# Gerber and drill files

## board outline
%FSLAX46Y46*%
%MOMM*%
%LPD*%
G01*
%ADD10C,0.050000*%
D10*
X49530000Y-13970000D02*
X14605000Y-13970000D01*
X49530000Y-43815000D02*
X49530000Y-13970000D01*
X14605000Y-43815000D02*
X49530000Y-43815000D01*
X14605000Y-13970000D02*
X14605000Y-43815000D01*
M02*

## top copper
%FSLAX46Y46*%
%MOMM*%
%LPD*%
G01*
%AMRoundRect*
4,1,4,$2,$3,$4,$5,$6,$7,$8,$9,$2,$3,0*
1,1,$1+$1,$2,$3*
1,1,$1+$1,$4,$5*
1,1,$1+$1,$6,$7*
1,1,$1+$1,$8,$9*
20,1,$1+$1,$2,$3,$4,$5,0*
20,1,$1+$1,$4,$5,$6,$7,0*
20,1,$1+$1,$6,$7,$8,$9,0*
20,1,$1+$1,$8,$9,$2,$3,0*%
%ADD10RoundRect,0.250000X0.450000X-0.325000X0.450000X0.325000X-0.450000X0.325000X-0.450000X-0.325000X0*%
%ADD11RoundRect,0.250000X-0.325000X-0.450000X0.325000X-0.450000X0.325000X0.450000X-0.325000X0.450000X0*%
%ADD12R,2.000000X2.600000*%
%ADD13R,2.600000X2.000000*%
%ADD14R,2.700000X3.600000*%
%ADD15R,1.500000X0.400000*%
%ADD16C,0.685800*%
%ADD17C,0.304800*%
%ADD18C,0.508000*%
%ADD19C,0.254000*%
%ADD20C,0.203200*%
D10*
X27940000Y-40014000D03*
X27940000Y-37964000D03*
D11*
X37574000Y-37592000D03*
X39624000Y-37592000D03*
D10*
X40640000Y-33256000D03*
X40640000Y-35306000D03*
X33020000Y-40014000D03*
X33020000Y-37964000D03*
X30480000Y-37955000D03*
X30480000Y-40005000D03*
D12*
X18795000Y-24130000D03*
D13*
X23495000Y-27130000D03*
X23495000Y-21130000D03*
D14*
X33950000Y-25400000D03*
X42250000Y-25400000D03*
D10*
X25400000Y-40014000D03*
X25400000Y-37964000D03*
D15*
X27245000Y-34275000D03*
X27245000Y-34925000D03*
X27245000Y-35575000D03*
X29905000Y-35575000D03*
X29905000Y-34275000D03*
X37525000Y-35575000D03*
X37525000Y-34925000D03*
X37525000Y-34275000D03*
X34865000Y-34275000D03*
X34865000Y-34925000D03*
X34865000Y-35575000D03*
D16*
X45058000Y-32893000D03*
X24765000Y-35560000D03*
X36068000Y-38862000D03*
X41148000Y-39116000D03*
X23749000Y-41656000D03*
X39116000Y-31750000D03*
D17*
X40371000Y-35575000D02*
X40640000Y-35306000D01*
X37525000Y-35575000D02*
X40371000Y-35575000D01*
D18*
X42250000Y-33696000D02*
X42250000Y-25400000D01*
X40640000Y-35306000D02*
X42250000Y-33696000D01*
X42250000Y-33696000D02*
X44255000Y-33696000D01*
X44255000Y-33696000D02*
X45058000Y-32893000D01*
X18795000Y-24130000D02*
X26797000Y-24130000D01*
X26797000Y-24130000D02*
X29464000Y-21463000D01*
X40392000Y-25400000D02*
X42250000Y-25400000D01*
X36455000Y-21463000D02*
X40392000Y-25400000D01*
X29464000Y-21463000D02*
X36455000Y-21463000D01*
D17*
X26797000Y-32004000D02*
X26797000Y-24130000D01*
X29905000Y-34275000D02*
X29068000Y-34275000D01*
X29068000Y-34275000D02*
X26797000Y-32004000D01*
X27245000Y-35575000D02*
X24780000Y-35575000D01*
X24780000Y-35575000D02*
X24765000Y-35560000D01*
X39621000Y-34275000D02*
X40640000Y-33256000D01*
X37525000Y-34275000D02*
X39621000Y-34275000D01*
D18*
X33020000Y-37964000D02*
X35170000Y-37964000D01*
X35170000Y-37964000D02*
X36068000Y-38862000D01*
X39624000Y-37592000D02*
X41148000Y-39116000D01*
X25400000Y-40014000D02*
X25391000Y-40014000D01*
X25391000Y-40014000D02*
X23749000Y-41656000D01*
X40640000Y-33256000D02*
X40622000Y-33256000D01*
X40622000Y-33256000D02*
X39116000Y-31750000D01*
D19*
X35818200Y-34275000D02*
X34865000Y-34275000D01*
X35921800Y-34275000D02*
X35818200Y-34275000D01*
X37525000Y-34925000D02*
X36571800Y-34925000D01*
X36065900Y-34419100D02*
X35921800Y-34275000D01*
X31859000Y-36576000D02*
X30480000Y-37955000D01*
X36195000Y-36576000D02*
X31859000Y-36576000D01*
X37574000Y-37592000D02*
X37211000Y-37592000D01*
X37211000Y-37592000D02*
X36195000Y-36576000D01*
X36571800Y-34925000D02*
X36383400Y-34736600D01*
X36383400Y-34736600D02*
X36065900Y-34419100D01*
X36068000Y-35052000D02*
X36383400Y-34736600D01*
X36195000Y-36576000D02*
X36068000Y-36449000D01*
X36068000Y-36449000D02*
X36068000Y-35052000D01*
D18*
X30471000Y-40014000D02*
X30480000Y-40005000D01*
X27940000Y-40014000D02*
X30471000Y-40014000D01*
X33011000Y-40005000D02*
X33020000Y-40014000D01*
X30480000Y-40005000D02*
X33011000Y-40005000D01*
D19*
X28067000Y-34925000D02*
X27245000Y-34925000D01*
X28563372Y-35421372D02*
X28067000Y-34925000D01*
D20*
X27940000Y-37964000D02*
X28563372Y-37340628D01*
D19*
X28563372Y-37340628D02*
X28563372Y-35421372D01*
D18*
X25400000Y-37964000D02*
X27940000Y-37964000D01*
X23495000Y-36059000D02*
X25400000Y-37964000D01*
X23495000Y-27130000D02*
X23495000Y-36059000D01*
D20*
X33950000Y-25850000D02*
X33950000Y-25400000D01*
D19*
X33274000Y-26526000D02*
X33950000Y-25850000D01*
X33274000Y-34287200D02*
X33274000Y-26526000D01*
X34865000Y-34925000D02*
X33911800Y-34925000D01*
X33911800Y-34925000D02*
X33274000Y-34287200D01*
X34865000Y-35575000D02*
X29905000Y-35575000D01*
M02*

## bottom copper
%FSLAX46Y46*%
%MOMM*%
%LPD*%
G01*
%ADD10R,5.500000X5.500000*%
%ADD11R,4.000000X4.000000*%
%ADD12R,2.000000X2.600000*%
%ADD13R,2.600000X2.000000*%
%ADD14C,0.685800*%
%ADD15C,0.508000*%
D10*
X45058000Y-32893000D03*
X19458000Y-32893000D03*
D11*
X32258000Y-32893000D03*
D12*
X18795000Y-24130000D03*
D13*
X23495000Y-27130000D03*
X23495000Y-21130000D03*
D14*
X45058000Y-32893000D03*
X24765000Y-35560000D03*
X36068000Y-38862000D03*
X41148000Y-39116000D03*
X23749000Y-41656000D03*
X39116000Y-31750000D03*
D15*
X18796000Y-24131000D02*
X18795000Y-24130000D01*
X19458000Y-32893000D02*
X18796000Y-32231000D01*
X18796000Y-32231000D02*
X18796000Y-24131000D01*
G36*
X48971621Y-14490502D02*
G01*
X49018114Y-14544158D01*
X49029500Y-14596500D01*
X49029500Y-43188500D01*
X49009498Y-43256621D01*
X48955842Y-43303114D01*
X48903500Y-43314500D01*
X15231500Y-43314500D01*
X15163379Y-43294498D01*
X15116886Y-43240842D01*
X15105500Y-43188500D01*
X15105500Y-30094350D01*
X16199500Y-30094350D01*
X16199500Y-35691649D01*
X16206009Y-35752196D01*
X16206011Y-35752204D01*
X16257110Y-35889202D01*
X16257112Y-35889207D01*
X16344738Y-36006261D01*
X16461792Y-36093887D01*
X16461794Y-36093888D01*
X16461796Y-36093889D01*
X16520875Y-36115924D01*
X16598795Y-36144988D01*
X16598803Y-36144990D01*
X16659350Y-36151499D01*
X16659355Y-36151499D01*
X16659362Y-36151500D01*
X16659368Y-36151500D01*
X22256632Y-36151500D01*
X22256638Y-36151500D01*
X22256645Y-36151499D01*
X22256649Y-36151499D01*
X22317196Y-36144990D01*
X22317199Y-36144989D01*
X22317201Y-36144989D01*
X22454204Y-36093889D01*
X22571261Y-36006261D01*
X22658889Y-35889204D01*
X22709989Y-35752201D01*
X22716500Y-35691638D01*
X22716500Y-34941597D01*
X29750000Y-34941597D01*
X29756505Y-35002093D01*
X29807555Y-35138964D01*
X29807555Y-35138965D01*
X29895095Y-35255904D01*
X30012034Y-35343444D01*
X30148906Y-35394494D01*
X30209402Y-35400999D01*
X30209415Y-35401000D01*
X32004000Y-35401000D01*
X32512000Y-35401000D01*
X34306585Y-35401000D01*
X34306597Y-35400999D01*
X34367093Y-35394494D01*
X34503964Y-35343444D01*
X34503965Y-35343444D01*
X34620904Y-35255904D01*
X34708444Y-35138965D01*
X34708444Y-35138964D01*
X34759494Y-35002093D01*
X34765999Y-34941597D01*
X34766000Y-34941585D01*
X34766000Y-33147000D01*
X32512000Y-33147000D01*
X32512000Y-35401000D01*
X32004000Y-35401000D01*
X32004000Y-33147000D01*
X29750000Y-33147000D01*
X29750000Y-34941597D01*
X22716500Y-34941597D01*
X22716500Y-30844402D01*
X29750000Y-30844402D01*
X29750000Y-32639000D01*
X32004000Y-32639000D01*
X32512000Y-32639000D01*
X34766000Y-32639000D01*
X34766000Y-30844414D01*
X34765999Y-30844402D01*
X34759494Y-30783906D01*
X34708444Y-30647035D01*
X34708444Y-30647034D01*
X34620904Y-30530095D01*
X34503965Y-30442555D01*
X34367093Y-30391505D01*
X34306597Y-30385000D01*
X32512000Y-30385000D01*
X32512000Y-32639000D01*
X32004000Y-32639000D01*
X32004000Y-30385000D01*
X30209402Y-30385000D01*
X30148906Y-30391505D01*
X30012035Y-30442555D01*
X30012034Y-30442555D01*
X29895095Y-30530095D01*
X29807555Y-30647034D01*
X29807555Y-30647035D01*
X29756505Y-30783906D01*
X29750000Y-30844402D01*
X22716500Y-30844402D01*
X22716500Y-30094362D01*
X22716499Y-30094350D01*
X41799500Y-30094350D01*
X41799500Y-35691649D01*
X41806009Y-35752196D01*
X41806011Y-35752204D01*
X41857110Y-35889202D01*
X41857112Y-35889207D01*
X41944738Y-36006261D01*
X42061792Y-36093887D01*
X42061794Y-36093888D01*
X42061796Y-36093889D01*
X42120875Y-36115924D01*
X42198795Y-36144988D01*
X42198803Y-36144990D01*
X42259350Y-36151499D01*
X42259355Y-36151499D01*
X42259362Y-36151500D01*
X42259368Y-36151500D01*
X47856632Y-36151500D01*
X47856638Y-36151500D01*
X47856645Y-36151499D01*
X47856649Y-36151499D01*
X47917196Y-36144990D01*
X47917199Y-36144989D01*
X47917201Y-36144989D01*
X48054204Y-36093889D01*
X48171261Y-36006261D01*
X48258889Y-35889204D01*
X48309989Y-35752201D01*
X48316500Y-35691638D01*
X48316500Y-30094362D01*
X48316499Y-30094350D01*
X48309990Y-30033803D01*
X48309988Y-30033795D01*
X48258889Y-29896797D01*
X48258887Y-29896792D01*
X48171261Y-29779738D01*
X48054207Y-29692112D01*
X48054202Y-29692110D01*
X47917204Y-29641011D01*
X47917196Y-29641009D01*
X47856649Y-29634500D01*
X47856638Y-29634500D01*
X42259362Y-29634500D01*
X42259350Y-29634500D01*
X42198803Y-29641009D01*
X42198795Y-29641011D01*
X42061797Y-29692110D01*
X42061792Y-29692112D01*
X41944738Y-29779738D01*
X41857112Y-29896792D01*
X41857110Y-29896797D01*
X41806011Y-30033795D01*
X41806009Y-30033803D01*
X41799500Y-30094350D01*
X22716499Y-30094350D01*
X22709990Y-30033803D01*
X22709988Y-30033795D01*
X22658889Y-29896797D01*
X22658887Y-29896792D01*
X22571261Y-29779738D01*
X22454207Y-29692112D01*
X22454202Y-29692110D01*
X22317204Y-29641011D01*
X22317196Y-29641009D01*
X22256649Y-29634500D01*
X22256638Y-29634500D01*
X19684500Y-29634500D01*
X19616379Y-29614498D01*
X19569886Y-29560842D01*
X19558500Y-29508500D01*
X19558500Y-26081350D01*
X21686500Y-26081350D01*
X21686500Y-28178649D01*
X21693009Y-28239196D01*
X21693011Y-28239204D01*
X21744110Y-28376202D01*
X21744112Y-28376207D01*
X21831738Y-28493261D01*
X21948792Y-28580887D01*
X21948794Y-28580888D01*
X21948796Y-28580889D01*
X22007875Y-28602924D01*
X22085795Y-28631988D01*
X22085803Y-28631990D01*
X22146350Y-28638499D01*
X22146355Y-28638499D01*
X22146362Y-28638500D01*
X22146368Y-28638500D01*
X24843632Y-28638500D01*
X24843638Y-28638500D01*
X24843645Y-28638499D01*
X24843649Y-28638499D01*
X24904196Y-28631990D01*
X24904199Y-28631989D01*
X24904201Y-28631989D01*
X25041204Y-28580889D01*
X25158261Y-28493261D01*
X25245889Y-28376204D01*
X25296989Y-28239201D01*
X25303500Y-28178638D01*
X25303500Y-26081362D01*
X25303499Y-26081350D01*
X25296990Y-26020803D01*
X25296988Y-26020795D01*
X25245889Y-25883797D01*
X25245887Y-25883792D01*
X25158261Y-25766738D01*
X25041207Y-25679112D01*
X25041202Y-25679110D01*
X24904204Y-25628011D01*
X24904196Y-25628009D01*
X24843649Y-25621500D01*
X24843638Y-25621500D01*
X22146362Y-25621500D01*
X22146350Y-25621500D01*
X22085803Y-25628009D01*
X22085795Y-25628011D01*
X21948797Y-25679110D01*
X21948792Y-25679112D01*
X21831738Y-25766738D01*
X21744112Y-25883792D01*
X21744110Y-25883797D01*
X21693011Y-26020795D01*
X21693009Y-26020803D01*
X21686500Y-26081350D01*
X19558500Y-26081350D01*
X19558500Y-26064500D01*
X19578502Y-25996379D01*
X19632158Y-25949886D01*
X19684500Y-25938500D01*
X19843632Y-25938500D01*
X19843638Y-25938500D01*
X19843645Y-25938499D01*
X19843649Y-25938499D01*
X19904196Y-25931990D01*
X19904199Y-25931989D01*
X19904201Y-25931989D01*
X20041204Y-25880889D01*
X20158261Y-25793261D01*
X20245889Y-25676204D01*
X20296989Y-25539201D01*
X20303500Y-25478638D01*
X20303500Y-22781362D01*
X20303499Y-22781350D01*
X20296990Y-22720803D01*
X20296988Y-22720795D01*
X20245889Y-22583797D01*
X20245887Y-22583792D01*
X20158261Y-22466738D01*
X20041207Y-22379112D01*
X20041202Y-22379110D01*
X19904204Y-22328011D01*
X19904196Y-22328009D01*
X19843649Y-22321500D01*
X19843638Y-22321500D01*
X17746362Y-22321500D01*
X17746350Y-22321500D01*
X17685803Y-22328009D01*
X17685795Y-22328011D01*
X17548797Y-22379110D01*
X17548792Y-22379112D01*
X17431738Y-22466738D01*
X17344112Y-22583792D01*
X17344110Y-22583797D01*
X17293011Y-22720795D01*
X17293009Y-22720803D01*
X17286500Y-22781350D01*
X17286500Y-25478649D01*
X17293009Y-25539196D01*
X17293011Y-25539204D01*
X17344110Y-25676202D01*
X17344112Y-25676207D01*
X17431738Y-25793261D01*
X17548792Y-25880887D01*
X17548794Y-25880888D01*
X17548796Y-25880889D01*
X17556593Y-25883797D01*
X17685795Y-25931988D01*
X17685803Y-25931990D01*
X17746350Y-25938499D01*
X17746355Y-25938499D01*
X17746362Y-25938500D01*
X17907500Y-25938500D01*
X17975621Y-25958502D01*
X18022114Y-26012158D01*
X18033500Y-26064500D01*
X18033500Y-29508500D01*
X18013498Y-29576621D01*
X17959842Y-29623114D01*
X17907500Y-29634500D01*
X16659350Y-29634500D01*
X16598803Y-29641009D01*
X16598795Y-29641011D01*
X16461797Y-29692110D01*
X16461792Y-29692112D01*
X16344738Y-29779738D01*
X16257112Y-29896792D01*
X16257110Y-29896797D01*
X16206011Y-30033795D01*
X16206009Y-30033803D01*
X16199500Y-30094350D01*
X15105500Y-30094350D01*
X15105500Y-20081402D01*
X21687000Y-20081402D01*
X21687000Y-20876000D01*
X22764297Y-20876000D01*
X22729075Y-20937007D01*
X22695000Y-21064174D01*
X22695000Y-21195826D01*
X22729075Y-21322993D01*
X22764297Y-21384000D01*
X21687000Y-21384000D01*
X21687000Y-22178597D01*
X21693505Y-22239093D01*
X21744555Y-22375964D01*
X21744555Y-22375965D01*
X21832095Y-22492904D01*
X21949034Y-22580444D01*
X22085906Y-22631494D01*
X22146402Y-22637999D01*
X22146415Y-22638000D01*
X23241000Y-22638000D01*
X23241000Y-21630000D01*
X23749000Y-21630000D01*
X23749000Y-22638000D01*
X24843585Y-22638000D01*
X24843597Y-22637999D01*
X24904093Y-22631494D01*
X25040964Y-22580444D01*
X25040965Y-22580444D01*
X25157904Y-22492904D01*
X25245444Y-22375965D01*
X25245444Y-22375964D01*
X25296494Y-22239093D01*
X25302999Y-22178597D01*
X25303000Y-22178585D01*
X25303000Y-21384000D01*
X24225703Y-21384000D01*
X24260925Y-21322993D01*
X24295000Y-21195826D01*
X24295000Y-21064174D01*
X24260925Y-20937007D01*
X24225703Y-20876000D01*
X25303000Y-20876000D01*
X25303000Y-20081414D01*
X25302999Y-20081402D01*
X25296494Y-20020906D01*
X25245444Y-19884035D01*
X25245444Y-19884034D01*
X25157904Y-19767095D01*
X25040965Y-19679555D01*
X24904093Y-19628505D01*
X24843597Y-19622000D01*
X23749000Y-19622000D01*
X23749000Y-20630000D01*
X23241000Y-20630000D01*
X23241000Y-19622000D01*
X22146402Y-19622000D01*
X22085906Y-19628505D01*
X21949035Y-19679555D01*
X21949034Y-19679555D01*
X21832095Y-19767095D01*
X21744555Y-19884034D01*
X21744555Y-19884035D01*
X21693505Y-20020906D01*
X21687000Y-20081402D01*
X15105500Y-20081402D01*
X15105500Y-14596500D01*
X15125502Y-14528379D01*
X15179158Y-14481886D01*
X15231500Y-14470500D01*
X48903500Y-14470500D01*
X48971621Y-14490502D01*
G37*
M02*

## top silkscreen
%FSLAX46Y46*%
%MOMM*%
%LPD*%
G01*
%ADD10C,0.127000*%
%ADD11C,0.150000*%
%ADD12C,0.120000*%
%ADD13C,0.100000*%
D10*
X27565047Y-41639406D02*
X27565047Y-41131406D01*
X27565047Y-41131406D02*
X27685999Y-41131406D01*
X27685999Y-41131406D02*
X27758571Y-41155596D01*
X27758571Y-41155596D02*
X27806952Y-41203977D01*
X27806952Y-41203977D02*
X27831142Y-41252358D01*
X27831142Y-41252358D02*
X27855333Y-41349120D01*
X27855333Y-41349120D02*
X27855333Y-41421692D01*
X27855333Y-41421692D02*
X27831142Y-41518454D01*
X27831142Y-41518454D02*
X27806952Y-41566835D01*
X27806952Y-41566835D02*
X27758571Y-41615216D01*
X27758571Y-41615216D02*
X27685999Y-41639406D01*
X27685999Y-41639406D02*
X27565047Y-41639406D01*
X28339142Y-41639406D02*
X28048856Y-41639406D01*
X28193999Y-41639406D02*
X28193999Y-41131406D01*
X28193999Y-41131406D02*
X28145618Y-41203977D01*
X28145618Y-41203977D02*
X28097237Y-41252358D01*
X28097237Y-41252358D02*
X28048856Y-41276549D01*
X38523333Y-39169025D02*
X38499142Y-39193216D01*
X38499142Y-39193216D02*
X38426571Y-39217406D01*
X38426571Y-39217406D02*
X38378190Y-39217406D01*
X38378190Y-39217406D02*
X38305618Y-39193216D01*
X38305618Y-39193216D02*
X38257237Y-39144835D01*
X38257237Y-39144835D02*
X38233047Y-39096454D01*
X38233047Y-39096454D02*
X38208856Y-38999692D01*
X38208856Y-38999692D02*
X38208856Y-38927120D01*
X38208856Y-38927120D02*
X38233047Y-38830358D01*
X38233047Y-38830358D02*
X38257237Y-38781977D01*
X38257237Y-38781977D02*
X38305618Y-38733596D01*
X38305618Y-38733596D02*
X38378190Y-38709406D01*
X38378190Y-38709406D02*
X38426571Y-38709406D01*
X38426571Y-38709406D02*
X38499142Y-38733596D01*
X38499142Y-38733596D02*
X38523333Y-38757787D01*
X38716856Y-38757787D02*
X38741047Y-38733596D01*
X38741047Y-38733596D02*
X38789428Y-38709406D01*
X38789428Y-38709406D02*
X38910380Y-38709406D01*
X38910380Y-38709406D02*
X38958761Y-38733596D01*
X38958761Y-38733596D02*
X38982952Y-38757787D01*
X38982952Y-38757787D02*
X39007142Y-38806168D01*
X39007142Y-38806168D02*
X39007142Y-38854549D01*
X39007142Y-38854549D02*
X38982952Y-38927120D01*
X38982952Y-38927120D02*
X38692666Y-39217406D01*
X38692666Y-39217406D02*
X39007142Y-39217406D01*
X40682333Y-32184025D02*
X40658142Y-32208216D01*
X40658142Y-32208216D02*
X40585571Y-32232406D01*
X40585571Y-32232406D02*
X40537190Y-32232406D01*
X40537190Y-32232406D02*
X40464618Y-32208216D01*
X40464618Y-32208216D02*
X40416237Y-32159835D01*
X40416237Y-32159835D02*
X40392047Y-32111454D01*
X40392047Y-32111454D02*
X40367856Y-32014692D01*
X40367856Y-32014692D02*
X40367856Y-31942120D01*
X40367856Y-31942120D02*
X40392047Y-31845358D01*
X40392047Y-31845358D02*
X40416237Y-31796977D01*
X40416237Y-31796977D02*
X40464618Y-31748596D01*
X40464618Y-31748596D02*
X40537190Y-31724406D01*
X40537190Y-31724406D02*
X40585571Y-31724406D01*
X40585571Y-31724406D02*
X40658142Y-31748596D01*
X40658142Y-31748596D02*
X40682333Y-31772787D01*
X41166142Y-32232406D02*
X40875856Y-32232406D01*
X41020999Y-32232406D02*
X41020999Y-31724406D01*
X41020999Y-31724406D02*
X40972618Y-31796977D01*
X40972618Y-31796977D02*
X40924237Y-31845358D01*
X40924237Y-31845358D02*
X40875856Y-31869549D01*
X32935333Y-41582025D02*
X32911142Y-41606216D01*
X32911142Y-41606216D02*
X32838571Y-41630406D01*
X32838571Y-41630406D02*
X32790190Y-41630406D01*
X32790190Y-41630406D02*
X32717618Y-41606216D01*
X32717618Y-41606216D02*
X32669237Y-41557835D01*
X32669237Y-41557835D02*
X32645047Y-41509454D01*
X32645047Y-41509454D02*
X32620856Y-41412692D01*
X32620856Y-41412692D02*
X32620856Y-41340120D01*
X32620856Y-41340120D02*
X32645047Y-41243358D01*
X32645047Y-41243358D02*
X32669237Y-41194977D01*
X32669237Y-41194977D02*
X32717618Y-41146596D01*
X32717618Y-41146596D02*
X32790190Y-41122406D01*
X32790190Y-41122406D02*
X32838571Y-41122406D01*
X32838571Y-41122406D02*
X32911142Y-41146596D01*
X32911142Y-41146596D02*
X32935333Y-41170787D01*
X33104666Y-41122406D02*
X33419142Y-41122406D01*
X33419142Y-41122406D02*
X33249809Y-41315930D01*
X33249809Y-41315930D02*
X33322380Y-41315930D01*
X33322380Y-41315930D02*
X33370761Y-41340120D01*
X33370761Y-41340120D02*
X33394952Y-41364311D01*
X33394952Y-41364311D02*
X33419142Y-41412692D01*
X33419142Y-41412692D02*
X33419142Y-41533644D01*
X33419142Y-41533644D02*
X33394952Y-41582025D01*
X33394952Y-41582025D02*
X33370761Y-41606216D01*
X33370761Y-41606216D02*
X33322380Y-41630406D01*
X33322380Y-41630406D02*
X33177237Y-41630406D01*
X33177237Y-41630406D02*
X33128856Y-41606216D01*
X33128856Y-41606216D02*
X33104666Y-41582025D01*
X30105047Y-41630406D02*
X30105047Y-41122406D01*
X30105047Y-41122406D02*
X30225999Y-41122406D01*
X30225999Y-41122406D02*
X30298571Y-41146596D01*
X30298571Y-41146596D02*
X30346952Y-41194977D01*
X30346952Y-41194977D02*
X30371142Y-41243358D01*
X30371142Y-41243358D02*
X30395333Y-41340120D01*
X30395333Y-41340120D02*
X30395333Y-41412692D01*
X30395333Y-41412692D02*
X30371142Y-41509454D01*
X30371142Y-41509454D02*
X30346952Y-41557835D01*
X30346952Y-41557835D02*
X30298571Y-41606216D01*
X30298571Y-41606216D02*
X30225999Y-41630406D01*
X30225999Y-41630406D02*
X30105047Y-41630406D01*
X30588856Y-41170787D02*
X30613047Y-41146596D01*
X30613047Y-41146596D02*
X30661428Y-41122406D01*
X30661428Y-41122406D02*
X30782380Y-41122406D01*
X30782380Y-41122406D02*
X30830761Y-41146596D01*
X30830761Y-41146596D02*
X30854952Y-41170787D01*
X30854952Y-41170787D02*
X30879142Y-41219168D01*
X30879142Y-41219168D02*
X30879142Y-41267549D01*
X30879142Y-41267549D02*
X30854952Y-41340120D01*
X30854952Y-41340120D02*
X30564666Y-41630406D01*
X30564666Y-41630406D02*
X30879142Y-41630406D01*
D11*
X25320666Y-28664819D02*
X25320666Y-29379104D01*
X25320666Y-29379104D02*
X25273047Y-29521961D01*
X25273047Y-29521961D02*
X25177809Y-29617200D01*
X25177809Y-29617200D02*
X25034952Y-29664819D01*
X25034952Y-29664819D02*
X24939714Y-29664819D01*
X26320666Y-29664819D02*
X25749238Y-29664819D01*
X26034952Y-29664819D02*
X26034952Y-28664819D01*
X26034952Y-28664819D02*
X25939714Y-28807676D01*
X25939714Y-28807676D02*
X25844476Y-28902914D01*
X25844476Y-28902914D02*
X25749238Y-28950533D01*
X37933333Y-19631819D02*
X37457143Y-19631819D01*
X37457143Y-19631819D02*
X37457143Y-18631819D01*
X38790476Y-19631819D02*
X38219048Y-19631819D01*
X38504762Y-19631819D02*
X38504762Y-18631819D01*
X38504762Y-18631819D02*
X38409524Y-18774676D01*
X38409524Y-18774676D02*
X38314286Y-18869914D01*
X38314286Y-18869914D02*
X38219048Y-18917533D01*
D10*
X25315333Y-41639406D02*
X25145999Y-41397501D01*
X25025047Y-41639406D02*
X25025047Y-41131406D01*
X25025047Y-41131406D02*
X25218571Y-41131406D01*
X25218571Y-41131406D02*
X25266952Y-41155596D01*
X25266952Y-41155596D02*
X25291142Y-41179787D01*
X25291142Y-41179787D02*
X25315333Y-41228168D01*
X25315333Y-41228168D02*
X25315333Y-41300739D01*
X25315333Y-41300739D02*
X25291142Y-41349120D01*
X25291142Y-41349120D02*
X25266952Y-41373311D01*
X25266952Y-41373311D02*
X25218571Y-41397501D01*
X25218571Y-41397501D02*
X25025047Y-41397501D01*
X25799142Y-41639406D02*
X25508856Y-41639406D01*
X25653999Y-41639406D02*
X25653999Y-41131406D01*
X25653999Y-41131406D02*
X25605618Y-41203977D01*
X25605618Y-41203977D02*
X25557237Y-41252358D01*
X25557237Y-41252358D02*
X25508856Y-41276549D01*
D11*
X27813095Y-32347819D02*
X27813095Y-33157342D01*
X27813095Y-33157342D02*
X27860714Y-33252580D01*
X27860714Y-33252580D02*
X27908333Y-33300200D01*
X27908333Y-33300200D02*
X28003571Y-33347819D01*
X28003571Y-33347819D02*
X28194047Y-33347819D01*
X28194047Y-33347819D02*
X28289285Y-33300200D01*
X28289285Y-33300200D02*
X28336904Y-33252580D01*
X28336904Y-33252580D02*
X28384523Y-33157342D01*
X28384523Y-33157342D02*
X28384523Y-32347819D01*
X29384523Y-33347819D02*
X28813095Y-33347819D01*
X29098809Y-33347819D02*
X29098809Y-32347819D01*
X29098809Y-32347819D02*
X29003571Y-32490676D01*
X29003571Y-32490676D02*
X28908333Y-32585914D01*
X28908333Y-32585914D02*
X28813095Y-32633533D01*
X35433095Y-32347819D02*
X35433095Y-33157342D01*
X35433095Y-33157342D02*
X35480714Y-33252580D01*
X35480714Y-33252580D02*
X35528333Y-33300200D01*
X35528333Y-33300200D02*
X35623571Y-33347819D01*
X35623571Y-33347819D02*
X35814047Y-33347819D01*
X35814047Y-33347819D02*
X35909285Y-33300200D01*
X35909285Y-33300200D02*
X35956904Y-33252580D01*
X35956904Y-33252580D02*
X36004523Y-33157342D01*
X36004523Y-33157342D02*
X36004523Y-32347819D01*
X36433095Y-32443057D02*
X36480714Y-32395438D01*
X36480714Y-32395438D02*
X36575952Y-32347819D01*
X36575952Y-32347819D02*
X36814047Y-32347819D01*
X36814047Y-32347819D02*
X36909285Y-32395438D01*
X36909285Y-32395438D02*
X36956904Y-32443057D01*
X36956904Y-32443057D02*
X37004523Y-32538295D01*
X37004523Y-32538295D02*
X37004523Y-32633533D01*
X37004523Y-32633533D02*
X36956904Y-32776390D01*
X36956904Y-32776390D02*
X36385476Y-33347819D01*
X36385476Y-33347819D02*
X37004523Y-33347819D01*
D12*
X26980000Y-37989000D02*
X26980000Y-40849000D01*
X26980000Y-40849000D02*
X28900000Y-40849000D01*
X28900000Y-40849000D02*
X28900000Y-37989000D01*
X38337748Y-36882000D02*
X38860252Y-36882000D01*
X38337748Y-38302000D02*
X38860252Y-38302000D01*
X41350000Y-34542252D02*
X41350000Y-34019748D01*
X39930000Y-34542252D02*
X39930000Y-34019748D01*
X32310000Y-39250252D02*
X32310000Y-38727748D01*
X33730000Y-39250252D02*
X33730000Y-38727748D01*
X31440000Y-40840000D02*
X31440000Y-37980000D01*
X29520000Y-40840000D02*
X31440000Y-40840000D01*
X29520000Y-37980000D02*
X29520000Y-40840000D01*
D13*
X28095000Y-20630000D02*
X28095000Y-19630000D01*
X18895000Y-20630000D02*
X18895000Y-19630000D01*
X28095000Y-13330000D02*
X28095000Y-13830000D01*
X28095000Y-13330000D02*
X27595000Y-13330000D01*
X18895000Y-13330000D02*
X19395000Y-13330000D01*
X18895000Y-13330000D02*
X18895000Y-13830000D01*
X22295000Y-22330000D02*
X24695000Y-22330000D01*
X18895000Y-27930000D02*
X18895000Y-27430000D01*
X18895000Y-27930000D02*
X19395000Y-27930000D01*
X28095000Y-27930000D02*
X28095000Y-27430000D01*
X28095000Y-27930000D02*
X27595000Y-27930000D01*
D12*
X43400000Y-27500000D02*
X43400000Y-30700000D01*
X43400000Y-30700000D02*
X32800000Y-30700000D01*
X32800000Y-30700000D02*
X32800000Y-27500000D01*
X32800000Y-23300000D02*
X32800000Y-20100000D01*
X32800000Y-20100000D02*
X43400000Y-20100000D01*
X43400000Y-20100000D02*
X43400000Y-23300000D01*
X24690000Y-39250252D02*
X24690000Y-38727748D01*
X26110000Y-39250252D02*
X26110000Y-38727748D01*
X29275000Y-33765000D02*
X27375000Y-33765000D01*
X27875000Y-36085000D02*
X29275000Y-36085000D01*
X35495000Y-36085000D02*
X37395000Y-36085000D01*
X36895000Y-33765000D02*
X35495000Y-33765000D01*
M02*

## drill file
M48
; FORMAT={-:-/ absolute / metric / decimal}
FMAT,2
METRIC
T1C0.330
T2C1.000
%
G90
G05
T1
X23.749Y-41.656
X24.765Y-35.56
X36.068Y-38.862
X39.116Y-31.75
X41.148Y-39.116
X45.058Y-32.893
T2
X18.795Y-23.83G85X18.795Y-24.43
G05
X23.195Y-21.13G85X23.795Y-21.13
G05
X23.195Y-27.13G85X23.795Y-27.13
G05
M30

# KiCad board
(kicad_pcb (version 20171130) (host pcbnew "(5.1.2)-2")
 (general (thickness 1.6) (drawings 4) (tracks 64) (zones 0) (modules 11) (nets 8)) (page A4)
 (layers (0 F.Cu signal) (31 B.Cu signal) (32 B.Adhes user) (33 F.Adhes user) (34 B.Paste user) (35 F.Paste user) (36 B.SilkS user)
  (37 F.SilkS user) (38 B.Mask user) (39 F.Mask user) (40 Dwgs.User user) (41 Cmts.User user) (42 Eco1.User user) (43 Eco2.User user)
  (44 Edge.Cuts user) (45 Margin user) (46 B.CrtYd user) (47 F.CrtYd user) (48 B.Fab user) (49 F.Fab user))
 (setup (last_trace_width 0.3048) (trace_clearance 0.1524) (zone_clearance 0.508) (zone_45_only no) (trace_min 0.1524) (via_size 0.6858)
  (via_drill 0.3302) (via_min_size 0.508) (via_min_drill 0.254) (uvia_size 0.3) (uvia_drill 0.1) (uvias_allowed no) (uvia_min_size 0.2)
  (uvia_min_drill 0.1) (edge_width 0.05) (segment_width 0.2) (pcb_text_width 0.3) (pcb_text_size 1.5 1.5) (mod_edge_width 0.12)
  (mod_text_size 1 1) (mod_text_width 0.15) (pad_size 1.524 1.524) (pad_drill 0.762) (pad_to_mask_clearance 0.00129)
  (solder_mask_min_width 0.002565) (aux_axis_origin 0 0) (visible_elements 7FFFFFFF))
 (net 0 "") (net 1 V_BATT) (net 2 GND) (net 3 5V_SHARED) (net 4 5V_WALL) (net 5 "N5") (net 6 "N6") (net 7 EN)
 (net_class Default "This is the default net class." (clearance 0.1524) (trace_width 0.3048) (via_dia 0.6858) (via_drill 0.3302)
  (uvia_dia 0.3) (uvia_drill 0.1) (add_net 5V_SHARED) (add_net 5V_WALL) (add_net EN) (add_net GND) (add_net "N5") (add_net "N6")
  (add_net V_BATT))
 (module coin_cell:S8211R (layer B.Cu) (at 32.258 32.893)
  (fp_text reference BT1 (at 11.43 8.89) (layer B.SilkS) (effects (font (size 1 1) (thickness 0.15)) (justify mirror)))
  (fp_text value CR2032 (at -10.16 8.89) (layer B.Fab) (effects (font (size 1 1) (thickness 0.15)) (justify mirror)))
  (pad 1 smd rect (at 12.8 0) (size 5.5 5.5) (layers B.Cu B.Paste B.Mask) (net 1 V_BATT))
  (pad 1 smd rect (at -12.8 0) (size 5.5 5.5) (layers B.Cu B.Paste B.Mask) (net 1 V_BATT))
  (pad 2 smd rect (at 0 0) (size 4 4) (layers B.Cu B.Paste B.Mask) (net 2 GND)))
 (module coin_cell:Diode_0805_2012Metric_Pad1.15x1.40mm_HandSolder (layer F.Cu) (at 27.94 38.989 90)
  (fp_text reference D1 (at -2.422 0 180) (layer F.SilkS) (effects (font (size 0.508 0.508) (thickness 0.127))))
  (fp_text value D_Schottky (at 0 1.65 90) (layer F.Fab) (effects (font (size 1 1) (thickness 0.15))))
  (fp_line (start 1 -0.96) (end -1.86 -0.96) (layer F.SilkS) (width 0.12))
  (fp_line (start -1.86 -0.96) (end -1.86 0.96) (layer F.SilkS) (width 0.12))
  (fp_line (start -1.86 0.96) (end 1 0.96) (layer F.SilkS) (width 0.12))
  (pad 1 smd roundrect (at -1.025 0 90) (size 1.15 1.4) (layers F.Cu F.Paste F.Mask) (roundrect_rratio 0.217391) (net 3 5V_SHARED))
  (pad 2 smd roundrect (at 1.025 0 90) (size 1.15 1.4) (layers F.Cu F.Paste F.Mask) (roundrect_rratio 0.217391) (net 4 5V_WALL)))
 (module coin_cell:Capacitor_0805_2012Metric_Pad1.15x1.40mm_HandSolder (layer F.Cu) (at 38.599 37.592)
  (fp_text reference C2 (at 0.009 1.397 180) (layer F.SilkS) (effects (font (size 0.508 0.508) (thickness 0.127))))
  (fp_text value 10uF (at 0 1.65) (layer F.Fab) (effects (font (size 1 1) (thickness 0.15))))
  (fp_line (start -0.261252 -0.71) (end 0.261252 -0.71) (layer F.SilkS) (width 0.12))
  (fp_line (start -0.261252 0.71) (end 0.261252 0.71) (layer F.SilkS) (width 0.12))
  (pad 1 smd roundrect (at -1.025 0) (size 1.15 1.4) (layers F.Cu F.Paste F.Mask) (roundrect_rratio 0.217391) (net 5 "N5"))
  (pad 2 smd roundrect (at 1.025 0) (size 1.15 1.4) (layers F.Cu F.Paste F.Mask) (roundrect_rratio 0.217391) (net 2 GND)))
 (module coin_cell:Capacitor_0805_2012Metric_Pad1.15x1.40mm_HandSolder (layer F.Cu) (at 40.64 34.281 90)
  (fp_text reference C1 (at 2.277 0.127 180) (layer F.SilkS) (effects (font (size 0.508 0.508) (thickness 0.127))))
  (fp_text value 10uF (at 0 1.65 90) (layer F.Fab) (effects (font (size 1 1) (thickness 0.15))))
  (fp_line (start -0.261252 0.71) (end 0.261252 0.71) (layer F.SilkS) (width 0.12))
  (fp_line (start -0.261252 -0.71) (end 0.261252 -0.71) (layer F.SilkS) (width 0.12))
  (pad 2 smd roundrect (at 1.025 0 90) (size 1.15 1.4) (layers F.Cu F.Paste F.Mask) (roundrect_rratio 0.217391) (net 2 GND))
  (pad 1 smd roundrect (at -1.025 0 90) (size 1.15 1.4) (layers F.Cu F.Paste F.Mask) (roundrect_rratio 0.217391) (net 1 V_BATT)))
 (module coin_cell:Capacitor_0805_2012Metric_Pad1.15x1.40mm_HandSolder (layer F.Cu) (at 33.02 38.989 90)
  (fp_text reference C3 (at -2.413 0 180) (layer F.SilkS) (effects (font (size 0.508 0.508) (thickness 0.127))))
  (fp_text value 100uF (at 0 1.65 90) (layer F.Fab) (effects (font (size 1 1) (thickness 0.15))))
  (fp_line (start -0.261252 -0.71) (end 0.261252 -0.71) (layer F.SilkS) (width 0.12))
  (fp_line (start -0.261252 0.71) (end 0.261252 0.71) (layer F.SilkS) (width 0.12))
  (pad 1 smd roundrect (at -1.025 0 90) (size 1.15 1.4) (layers F.Cu F.Paste F.Mask) (roundrect_rratio 0.217391) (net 3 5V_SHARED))
  (pad 2 smd roundrect (at 1.025 0 90) (size 1.15 1.4) (layers F.Cu F.Paste F.Mask) (roundrect_rratio 0.217391) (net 2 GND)))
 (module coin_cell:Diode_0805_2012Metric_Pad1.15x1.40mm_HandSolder (layer F.Cu) (at 30.48 38.98 90)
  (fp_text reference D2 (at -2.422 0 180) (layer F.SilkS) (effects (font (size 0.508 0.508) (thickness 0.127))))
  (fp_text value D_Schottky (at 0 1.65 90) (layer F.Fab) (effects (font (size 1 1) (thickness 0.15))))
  (fp_line (start -1.86 0.96) (end 1 0.96) (layer F.SilkS) (width 0.12))
  (fp_line (start -1.86 -0.96) (end -1.86 0.96) (layer F.SilkS) (width 0.12))
  (fp_line (start 1 -0.96) (end -1.86 -0.96) (layer F.SilkS) (width 0.12))
  (pad 2 smd roundrect (at 1.025 0 90) (size 1.15 1.4) (layers F.Cu F.Paste F.Mask) (roundrect_rratio 0.217391) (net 5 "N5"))
  (pad 1 smd roundrect (at -1.025 0 90) (size 1.15 1.4) (layers F.Cu F.Paste F.Mask) (roundrect_rratio 0.217391) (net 3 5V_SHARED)))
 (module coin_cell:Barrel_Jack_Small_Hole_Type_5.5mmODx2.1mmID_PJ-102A (layer F.Cu) (at 23.495 24.13)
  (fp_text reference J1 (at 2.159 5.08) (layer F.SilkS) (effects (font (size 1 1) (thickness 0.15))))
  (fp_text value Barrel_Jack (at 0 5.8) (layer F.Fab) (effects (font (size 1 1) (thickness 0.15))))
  (fp_line (start 4.6 -3.5) (end 4.6 -4.5) (layer F.SilkS) (width 0.1))
  (fp_line (start -4.6 -3.5) (end -4.6 -4.5) (layer F.SilkS) (width 0.1))
  (fp_line (start 4.6 -10.8) (end 4.6 -10.3) (layer F.SilkS) (width 0.1))
  (fp_line (start 4.6 -10.8) (end 4.1 -10.8) (layer F.SilkS) (width 0.1))
  (fp_line (start -4.6 -10.8) (end -4.1 -10.8) (layer F.SilkS) (width 0.1))
  (fp_line (start -4.6 -10.8) (end -4.6 -10.3) (layer F.SilkS) (width 0.1))
  (fp_line (start -1.2 -1.8) (end 1.2 -1.8) (layer F.SilkS) (width 0.1))
  (fp_line (start -4.6 3.8) (end -4.6 3.3) (layer F.SilkS) (width 0.1))
  (fp_line (start -4.6 3.8) (end -4.1 3.8) (layer F.SilkS) (width 0.1))
  (fp_line (start 4.6 3.8) (end 4.6 3.3) (layer F.SilkS) (width 0.1))
  (fp_line (start 4.6 3.8) (end 4.1 3.8) (layer F.SilkS) (width 0.1))
  (pad 3 thru_hole rect (at -4.7 0) (size 2 2.6) (drill oval 1 1.6) (layers *.Cu *.Mask) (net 1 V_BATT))
  (pad 1 thru_hole rect (at 0 3) (size 2.6 2) (drill oval 1.6 1) (layers *.Cu *.Mask) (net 4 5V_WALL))
  (pad 2 thru_hole rect (at 0 -3) (size 2.6 2) (drill oval 1.6 1) (layers *.Cu *.Mask) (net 2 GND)))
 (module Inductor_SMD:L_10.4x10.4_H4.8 (layer F.Cu) (at 38.1 25.4)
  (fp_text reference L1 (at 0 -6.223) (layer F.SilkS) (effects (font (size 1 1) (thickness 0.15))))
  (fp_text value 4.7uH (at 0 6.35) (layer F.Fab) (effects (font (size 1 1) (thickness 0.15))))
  (fp_line (start 5.3 2.1) (end 5.3 5.3) (layer F.SilkS) (width 0.12))
  (fp_line (start 5.3 5.3) (end -5.3 5.3) (layer F.SilkS) (width 0.12))
  (fp_line (start -5.3 5.3) (end -5.3 2.1) (layer F.SilkS) (width 0.12))
  (fp_line (start -5.3 -2.1) (end -5.3 -5.3) (layer F.SilkS) (width 0.12))
  (fp_line (start -5.3 -5.3) (end 5.3 -5.3) (layer F.SilkS) (width 0.12))
  (fp_line (start 5.3 -5.3) (end 5.3 -2.1) (layer F.SilkS) (width 0.12))
  (pad 1 smd rect (at -4.15 0) (size 2.7 3.6) (layers F.Cu F.Paste F.Mask) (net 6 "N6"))
  (pad 2 smd rect (at 4.15 0) (size 2.7 3.6) (layers F.Cu F.Paste F.Mask) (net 1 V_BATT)))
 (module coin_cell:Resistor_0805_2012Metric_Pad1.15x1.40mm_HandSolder (layer F.Cu) (at 25.4 38.989 90)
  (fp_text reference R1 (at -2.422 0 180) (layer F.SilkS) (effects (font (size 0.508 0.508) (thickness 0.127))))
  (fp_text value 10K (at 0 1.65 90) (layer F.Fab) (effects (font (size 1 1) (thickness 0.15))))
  (fp_line (start -0.261252 -0.71) (end 0.261252 -0.71) (layer F.SilkS) (width 0.12))
  (fp_line (start -0.261252 0.71) (end 0.261252 0.71) (layer F.SilkS) (width 0.12))
  (pad 1 smd roundrect (at -1.025 0 90) (size 1.15 1.4) (layers F.Cu F.Paste F.Mask) (roundrect_rratio 0.217391) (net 2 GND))
  (pad 2 smd roundrect (at 1.025 0 90) (size 1.15 1.4) (layers F.Cu F.Paste F.Mask) (roundrect_rratio 0.217391) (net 4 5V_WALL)))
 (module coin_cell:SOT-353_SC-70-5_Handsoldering (layer F.Cu) (at 28.575 34.925)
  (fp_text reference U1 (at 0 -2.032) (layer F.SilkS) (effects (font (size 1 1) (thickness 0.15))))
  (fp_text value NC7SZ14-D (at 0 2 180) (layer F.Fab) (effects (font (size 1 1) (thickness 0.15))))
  (fp_line (start 0.7 -1.16) (end -1.2 -1.16) (layer F.SilkS) (width 0.12))
  (fp_line (start -0.7 1.16) (end 0.7 1.16) (layer F.SilkS) (width 0.12))
  (pad 1 smd rect (at -1.33 -0.65) (size 1.5 0.4) (layers F.Cu F.Paste F.Mask))
  (pad 2 smd rect (at -1.33 0) (size 1.5 0.4) (layers F.Cu F.Paste F.Mask) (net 4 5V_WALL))
  (pad 3 smd rect (at -1.33 0.65) (size 1.5 0.4) (layers F.Cu F.Paste F.Mask) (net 2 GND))
  (pad 4 smd rect (at 1.33 0.65) (size 1.5 0.4) (layers F.Cu F.Paste F.Mask) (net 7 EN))
  (pad 5 smd rect (at 1.33 -0.65) (size 1.5 0.4) (layers F.Cu F.Paste F.Mask) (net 1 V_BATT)))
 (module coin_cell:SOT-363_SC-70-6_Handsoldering (layer F.Cu) (at 36.195 34.925 180)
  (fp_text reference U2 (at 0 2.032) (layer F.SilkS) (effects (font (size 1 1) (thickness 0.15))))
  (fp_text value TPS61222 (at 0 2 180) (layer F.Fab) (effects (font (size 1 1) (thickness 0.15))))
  (fp_line (start 0.7 -1.16) (end -1.2 -1.16) (layer F.SilkS) (width 0.12))
  (fp_line (start -0.7 1.16) (end 0.7 1.16) (layer F.SilkS) (width 0.12))
  (pad 1 smd rect (at -1.33 -0.65 180) (size 1.5 0.4) (layers F.Cu F.Paste F.Mask) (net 1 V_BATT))
  (pad 2 smd rect (at -1.33 0 180) (size 1.5 0.4) (layers F.Cu F.Paste F.Mask) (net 5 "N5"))
  (pad 3 smd rect (at -1.33 0.65 180) (size 1.5 0.4) (layers F.Cu F.Paste F.Mask) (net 2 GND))
  (pad 4 smd rect (at 1.33 0.65 180) (size 1.5 0.4) (layers F.Cu F.Paste F.Mask) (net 5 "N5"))
  (pad 5 smd rect (at 1.33 0 180) (size 1.5 0.4) (layers F.Cu F.Paste F.Mask) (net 6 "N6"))
  (pad 6 smd rect (at 1.33 -0.65 180) (size 1.5 0.4) (layers F.Cu F.Paste F.Mask) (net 7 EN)))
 (gr_line (start 49.53 13.97) (end 14.605 13.97) (layer Edge.Cuts) (width 0.05))
 (gr_line (start 49.53 43.815) (end 49.53 13.97) (layer Edge.Cuts) (width 0.05))
 (gr_line (start 14.605 43.815) (end 49.53 43.815) (layer Edge.Cuts) (width 0.05))
 (gr_line (start 14.605 13.97) (end 14.605 43.815) (layer Edge.Cuts) (width 0.05))
 (segment (start 40.371 35.575) (end 40.64 35.306) (width 0.3048) (layer F.Cu) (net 1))
 (segment (start 37.525 35.575) (end 40.371 35.575) (width 0.3048) (layer F.Cu) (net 1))
 (segment (start 42.25 33.696) (end 42.25 25.4) (width 0.508) (layer F.Cu) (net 1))
 (segment (start 40.64 35.306) (end 42.25 33.696) (width 0.508) (layer F.Cu) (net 1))
 (segment (start 18.796 24.131) (end 18.795 24.13) (width 0.508) (layer B.Cu) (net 1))
 (segment (start 19.458 32.893) (end 18.796 32.231) (width 0.508) (layer B.Cu) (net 1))
 (segment (start 18.796 32.231) (end 18.796 24.131) (width 0.508) (layer B.Cu) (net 1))
 (via (at 45.058 32.893) (size 0.6858) (drill 0.3302) (layers F.Cu B.Cu) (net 1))
 (segment (start 42.25 33.696) (end 44.255 33.696) (width 0.508) (layer F.Cu) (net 1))
 (segment (start 44.255 33.696) (end 45.058 32.893) (width 0.508) (layer F.Cu) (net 1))
 (segment (start 18.795 24.13) (end 26.797 24.13) (width 0.508) (layer F.Cu) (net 1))
 (segment (start 26.797 24.13) (end 29.464 21.463) (width 0.508) (layer F.Cu) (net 1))
 (segment (start 40.392 25.4) (end 42.25 25.4) (width 0.508) (layer F.Cu) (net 1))
 (segment (start 36.455 21.463) (end 40.392 25.4) (width 0.508) (layer F.Cu) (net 1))
 (segment (start 29.464 21.463) (end 36.455 21.463) (width 0.508) (layer F.Cu) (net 1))
 (segment (start 26.797 32.004) (end 26.797 24.13) (width 0.3048) (layer F.Cu) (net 1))
 (segment (start 29.905 34.275) (end 29.068 34.275) (width 0.3048) (layer F.Cu) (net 1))
 (segment (start 29.068 34.275) (end 26.797 32.004) (width 0.3048) (layer F.Cu) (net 1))
 (via (at 24.765 35.56) (size 0.6858) (drill 0.3302) (layers F.Cu B.Cu) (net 2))
 (segment (start 27.245 35.575) (end 24.78 35.575) (width 0.3048) (layer F.Cu) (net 2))
 (segment (start 24.78 35.575) (end 24.765 35.56) (width 0.3048) (layer F.Cu) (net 2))
 (segment (start 39.621 34.275) (end 40.64 33.256) (width 0.3048) (layer F.Cu) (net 2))
 (segment (start 37.525 34.275) (end 39.621 34.275) (width 0.3048) (layer F.Cu) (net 2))
 (via (at 36.068 38.862) (size 0.6858) (drill 0.3302) (layers F.Cu B.Cu) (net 2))
 (segment (start 33.02 37.964) (end 35.17 37.964) (width 0.508) (layer F.Cu) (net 2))
 (segment (start 35.17 37.964) (end 36.068 38.862) (width 0.508) (layer F.Cu) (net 2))
 (via (at 41.148 39.116) (size 0.6858) (drill 0.3302) (layers F.Cu B.Cu) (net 2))
 (segment (start 39.624 37.592) (end 41.148 39.116) (width 0.508) (layer F.Cu) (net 2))
 (via (at 23.749 41.656) (size 0.6858) (drill 0.3302) (layers F.Cu B.Cu) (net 2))
 (segment (start 25.4 40.014) (end 25.391 40.014) (width 0.508) (layer F.Cu) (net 2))
 (segment (start 25.391 40.014) (end 23.749 41.656) (width 0.508) (layer F.Cu) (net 2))
 (via (at 39.116 31.75) (size 0.6858) (drill 0.3302) (layers F.Cu B.Cu) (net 2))
 (segment (start 40.64 33.256) (end 40.622 33.256) (width 0.508) (layer F.Cu) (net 2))
 (segment (start 40.622 33.256) (end 39.116 31.75) (width 0.508) (layer F.Cu) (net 2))
 (segment (start 35.8182 34.275) (end 34.865 34.275) (width 0.254) (layer F.Cu) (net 5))
 (segment (start 35.9218 34.275) (end 35.8182 34.275) (width 0.254) (layer F.Cu) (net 5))
 (segment (start 37.525 34.925) (end 36.5718 34.925) (width 0.254) (layer F.Cu) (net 5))
 (segment (start 36.0659 34.4191) (end 35.9218 34.275) (width 0.254) (layer F.Cu) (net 5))
 (segment (start 31.859 36.576) (end 30.48 37.955) (width 0.254) (layer F.Cu) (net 5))
 (segment (start 36.195 36.576) (end 31.859 36.576) (width 0.254) (layer F.Cu) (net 5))
 (segment (start 37.574 37.592) (end 37.211 37.592) (width 0.254) (layer F.Cu) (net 5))
 (segment (start 37.211 37.592) (end 36.195 36.576) (width 0.254) (layer F.Cu) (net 5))
 (segment (start 36.5718 34.925) (end 36.3834 34.7366) (width 0.254) (layer F.Cu) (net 5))
 (segment (start 36.3834 34.7366) (end 36.0659 34.4191) (width 0.254) (layer F.Cu) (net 5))
 (segment (start 36.068 35.052) (end 36.3834 34.7366) (width 0.254) (layer F.Cu) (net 5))
 (segment (start 36.195 36.576) (end 36.068 36.449) (width 0.254) (layer F.Cu) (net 5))
 (segment (start 36.068 36.449) (end 36.068 35.052) (width 0.254) (layer F.Cu) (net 5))
 (segment (start 30.471 40.014) (end 30.48 40.005) (width 0.508) (layer F.Cu) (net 3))
 (segment (start 27.94 40.014) (end 30.471 40.014) (width 0.508) (layer F.Cu) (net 3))
 (segment (start 33.011 40.005) (end 33.02 40.014) (width 0.508) (layer F.Cu) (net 3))
 (segment (start 30.48 40.005) (end 33.011 40.005) (width 0.508) (layer F.Cu) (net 3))
 (segment (start 28.067 34.925) (end 27.245 34.925) (width 0.254) (layer F.Cu) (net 4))
 (segment (start 28.563372 35.421372) (end 28.067 34.925) (width 0.254) (layer F.Cu) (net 4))
 (segment (start 27.94 37.964) (end 28.563372 37.340628) (width 0.2032) (layer F.Cu) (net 4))
 (segment (start 28.563372 37.340628) (end 28.563372 35.421372) (width 0.254) (layer F.Cu) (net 4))
 (segment (start 25.4 37.964) (end 27.94 37.964) (width 0.508) (layer F.Cu) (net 4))
 (segment (start 23.495 36.059) (end 25.4 37.964) (width 0.508) (layer F.Cu) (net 4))
 (segment (start 23.495 27.13) (end 23.495 36.059) (width 0.508) (layer F.Cu) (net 4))
 (segment (start 33.95 25.85) (end 33.95 25.4) (width 0.2032) (layer F.Cu) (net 6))
 (segment (start 33.274 26.526) (end 33.95 25.85) (width 0.254) (layer F.Cu) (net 6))
 (segment (start 33.274 34.2872) (end 33.274 26.526) (width 0.254) (layer F.Cu) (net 6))
 (segment (start 34.865 34.925) (end 33.9118 34.925) (width 0.254) (layer F.Cu) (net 6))
 (segment (start 33.9118 34.925) (end 33.274 34.2872) (width 0.254) (layer F.Cu) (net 6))
 (segment (start 34.865 35.575) (end 29.905 35.575) (width 0.254) (layer F.Cu) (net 7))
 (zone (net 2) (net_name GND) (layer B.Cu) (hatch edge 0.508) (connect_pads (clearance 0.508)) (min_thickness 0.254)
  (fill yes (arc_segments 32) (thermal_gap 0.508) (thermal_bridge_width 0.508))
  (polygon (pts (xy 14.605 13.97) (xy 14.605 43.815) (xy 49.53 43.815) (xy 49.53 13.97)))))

